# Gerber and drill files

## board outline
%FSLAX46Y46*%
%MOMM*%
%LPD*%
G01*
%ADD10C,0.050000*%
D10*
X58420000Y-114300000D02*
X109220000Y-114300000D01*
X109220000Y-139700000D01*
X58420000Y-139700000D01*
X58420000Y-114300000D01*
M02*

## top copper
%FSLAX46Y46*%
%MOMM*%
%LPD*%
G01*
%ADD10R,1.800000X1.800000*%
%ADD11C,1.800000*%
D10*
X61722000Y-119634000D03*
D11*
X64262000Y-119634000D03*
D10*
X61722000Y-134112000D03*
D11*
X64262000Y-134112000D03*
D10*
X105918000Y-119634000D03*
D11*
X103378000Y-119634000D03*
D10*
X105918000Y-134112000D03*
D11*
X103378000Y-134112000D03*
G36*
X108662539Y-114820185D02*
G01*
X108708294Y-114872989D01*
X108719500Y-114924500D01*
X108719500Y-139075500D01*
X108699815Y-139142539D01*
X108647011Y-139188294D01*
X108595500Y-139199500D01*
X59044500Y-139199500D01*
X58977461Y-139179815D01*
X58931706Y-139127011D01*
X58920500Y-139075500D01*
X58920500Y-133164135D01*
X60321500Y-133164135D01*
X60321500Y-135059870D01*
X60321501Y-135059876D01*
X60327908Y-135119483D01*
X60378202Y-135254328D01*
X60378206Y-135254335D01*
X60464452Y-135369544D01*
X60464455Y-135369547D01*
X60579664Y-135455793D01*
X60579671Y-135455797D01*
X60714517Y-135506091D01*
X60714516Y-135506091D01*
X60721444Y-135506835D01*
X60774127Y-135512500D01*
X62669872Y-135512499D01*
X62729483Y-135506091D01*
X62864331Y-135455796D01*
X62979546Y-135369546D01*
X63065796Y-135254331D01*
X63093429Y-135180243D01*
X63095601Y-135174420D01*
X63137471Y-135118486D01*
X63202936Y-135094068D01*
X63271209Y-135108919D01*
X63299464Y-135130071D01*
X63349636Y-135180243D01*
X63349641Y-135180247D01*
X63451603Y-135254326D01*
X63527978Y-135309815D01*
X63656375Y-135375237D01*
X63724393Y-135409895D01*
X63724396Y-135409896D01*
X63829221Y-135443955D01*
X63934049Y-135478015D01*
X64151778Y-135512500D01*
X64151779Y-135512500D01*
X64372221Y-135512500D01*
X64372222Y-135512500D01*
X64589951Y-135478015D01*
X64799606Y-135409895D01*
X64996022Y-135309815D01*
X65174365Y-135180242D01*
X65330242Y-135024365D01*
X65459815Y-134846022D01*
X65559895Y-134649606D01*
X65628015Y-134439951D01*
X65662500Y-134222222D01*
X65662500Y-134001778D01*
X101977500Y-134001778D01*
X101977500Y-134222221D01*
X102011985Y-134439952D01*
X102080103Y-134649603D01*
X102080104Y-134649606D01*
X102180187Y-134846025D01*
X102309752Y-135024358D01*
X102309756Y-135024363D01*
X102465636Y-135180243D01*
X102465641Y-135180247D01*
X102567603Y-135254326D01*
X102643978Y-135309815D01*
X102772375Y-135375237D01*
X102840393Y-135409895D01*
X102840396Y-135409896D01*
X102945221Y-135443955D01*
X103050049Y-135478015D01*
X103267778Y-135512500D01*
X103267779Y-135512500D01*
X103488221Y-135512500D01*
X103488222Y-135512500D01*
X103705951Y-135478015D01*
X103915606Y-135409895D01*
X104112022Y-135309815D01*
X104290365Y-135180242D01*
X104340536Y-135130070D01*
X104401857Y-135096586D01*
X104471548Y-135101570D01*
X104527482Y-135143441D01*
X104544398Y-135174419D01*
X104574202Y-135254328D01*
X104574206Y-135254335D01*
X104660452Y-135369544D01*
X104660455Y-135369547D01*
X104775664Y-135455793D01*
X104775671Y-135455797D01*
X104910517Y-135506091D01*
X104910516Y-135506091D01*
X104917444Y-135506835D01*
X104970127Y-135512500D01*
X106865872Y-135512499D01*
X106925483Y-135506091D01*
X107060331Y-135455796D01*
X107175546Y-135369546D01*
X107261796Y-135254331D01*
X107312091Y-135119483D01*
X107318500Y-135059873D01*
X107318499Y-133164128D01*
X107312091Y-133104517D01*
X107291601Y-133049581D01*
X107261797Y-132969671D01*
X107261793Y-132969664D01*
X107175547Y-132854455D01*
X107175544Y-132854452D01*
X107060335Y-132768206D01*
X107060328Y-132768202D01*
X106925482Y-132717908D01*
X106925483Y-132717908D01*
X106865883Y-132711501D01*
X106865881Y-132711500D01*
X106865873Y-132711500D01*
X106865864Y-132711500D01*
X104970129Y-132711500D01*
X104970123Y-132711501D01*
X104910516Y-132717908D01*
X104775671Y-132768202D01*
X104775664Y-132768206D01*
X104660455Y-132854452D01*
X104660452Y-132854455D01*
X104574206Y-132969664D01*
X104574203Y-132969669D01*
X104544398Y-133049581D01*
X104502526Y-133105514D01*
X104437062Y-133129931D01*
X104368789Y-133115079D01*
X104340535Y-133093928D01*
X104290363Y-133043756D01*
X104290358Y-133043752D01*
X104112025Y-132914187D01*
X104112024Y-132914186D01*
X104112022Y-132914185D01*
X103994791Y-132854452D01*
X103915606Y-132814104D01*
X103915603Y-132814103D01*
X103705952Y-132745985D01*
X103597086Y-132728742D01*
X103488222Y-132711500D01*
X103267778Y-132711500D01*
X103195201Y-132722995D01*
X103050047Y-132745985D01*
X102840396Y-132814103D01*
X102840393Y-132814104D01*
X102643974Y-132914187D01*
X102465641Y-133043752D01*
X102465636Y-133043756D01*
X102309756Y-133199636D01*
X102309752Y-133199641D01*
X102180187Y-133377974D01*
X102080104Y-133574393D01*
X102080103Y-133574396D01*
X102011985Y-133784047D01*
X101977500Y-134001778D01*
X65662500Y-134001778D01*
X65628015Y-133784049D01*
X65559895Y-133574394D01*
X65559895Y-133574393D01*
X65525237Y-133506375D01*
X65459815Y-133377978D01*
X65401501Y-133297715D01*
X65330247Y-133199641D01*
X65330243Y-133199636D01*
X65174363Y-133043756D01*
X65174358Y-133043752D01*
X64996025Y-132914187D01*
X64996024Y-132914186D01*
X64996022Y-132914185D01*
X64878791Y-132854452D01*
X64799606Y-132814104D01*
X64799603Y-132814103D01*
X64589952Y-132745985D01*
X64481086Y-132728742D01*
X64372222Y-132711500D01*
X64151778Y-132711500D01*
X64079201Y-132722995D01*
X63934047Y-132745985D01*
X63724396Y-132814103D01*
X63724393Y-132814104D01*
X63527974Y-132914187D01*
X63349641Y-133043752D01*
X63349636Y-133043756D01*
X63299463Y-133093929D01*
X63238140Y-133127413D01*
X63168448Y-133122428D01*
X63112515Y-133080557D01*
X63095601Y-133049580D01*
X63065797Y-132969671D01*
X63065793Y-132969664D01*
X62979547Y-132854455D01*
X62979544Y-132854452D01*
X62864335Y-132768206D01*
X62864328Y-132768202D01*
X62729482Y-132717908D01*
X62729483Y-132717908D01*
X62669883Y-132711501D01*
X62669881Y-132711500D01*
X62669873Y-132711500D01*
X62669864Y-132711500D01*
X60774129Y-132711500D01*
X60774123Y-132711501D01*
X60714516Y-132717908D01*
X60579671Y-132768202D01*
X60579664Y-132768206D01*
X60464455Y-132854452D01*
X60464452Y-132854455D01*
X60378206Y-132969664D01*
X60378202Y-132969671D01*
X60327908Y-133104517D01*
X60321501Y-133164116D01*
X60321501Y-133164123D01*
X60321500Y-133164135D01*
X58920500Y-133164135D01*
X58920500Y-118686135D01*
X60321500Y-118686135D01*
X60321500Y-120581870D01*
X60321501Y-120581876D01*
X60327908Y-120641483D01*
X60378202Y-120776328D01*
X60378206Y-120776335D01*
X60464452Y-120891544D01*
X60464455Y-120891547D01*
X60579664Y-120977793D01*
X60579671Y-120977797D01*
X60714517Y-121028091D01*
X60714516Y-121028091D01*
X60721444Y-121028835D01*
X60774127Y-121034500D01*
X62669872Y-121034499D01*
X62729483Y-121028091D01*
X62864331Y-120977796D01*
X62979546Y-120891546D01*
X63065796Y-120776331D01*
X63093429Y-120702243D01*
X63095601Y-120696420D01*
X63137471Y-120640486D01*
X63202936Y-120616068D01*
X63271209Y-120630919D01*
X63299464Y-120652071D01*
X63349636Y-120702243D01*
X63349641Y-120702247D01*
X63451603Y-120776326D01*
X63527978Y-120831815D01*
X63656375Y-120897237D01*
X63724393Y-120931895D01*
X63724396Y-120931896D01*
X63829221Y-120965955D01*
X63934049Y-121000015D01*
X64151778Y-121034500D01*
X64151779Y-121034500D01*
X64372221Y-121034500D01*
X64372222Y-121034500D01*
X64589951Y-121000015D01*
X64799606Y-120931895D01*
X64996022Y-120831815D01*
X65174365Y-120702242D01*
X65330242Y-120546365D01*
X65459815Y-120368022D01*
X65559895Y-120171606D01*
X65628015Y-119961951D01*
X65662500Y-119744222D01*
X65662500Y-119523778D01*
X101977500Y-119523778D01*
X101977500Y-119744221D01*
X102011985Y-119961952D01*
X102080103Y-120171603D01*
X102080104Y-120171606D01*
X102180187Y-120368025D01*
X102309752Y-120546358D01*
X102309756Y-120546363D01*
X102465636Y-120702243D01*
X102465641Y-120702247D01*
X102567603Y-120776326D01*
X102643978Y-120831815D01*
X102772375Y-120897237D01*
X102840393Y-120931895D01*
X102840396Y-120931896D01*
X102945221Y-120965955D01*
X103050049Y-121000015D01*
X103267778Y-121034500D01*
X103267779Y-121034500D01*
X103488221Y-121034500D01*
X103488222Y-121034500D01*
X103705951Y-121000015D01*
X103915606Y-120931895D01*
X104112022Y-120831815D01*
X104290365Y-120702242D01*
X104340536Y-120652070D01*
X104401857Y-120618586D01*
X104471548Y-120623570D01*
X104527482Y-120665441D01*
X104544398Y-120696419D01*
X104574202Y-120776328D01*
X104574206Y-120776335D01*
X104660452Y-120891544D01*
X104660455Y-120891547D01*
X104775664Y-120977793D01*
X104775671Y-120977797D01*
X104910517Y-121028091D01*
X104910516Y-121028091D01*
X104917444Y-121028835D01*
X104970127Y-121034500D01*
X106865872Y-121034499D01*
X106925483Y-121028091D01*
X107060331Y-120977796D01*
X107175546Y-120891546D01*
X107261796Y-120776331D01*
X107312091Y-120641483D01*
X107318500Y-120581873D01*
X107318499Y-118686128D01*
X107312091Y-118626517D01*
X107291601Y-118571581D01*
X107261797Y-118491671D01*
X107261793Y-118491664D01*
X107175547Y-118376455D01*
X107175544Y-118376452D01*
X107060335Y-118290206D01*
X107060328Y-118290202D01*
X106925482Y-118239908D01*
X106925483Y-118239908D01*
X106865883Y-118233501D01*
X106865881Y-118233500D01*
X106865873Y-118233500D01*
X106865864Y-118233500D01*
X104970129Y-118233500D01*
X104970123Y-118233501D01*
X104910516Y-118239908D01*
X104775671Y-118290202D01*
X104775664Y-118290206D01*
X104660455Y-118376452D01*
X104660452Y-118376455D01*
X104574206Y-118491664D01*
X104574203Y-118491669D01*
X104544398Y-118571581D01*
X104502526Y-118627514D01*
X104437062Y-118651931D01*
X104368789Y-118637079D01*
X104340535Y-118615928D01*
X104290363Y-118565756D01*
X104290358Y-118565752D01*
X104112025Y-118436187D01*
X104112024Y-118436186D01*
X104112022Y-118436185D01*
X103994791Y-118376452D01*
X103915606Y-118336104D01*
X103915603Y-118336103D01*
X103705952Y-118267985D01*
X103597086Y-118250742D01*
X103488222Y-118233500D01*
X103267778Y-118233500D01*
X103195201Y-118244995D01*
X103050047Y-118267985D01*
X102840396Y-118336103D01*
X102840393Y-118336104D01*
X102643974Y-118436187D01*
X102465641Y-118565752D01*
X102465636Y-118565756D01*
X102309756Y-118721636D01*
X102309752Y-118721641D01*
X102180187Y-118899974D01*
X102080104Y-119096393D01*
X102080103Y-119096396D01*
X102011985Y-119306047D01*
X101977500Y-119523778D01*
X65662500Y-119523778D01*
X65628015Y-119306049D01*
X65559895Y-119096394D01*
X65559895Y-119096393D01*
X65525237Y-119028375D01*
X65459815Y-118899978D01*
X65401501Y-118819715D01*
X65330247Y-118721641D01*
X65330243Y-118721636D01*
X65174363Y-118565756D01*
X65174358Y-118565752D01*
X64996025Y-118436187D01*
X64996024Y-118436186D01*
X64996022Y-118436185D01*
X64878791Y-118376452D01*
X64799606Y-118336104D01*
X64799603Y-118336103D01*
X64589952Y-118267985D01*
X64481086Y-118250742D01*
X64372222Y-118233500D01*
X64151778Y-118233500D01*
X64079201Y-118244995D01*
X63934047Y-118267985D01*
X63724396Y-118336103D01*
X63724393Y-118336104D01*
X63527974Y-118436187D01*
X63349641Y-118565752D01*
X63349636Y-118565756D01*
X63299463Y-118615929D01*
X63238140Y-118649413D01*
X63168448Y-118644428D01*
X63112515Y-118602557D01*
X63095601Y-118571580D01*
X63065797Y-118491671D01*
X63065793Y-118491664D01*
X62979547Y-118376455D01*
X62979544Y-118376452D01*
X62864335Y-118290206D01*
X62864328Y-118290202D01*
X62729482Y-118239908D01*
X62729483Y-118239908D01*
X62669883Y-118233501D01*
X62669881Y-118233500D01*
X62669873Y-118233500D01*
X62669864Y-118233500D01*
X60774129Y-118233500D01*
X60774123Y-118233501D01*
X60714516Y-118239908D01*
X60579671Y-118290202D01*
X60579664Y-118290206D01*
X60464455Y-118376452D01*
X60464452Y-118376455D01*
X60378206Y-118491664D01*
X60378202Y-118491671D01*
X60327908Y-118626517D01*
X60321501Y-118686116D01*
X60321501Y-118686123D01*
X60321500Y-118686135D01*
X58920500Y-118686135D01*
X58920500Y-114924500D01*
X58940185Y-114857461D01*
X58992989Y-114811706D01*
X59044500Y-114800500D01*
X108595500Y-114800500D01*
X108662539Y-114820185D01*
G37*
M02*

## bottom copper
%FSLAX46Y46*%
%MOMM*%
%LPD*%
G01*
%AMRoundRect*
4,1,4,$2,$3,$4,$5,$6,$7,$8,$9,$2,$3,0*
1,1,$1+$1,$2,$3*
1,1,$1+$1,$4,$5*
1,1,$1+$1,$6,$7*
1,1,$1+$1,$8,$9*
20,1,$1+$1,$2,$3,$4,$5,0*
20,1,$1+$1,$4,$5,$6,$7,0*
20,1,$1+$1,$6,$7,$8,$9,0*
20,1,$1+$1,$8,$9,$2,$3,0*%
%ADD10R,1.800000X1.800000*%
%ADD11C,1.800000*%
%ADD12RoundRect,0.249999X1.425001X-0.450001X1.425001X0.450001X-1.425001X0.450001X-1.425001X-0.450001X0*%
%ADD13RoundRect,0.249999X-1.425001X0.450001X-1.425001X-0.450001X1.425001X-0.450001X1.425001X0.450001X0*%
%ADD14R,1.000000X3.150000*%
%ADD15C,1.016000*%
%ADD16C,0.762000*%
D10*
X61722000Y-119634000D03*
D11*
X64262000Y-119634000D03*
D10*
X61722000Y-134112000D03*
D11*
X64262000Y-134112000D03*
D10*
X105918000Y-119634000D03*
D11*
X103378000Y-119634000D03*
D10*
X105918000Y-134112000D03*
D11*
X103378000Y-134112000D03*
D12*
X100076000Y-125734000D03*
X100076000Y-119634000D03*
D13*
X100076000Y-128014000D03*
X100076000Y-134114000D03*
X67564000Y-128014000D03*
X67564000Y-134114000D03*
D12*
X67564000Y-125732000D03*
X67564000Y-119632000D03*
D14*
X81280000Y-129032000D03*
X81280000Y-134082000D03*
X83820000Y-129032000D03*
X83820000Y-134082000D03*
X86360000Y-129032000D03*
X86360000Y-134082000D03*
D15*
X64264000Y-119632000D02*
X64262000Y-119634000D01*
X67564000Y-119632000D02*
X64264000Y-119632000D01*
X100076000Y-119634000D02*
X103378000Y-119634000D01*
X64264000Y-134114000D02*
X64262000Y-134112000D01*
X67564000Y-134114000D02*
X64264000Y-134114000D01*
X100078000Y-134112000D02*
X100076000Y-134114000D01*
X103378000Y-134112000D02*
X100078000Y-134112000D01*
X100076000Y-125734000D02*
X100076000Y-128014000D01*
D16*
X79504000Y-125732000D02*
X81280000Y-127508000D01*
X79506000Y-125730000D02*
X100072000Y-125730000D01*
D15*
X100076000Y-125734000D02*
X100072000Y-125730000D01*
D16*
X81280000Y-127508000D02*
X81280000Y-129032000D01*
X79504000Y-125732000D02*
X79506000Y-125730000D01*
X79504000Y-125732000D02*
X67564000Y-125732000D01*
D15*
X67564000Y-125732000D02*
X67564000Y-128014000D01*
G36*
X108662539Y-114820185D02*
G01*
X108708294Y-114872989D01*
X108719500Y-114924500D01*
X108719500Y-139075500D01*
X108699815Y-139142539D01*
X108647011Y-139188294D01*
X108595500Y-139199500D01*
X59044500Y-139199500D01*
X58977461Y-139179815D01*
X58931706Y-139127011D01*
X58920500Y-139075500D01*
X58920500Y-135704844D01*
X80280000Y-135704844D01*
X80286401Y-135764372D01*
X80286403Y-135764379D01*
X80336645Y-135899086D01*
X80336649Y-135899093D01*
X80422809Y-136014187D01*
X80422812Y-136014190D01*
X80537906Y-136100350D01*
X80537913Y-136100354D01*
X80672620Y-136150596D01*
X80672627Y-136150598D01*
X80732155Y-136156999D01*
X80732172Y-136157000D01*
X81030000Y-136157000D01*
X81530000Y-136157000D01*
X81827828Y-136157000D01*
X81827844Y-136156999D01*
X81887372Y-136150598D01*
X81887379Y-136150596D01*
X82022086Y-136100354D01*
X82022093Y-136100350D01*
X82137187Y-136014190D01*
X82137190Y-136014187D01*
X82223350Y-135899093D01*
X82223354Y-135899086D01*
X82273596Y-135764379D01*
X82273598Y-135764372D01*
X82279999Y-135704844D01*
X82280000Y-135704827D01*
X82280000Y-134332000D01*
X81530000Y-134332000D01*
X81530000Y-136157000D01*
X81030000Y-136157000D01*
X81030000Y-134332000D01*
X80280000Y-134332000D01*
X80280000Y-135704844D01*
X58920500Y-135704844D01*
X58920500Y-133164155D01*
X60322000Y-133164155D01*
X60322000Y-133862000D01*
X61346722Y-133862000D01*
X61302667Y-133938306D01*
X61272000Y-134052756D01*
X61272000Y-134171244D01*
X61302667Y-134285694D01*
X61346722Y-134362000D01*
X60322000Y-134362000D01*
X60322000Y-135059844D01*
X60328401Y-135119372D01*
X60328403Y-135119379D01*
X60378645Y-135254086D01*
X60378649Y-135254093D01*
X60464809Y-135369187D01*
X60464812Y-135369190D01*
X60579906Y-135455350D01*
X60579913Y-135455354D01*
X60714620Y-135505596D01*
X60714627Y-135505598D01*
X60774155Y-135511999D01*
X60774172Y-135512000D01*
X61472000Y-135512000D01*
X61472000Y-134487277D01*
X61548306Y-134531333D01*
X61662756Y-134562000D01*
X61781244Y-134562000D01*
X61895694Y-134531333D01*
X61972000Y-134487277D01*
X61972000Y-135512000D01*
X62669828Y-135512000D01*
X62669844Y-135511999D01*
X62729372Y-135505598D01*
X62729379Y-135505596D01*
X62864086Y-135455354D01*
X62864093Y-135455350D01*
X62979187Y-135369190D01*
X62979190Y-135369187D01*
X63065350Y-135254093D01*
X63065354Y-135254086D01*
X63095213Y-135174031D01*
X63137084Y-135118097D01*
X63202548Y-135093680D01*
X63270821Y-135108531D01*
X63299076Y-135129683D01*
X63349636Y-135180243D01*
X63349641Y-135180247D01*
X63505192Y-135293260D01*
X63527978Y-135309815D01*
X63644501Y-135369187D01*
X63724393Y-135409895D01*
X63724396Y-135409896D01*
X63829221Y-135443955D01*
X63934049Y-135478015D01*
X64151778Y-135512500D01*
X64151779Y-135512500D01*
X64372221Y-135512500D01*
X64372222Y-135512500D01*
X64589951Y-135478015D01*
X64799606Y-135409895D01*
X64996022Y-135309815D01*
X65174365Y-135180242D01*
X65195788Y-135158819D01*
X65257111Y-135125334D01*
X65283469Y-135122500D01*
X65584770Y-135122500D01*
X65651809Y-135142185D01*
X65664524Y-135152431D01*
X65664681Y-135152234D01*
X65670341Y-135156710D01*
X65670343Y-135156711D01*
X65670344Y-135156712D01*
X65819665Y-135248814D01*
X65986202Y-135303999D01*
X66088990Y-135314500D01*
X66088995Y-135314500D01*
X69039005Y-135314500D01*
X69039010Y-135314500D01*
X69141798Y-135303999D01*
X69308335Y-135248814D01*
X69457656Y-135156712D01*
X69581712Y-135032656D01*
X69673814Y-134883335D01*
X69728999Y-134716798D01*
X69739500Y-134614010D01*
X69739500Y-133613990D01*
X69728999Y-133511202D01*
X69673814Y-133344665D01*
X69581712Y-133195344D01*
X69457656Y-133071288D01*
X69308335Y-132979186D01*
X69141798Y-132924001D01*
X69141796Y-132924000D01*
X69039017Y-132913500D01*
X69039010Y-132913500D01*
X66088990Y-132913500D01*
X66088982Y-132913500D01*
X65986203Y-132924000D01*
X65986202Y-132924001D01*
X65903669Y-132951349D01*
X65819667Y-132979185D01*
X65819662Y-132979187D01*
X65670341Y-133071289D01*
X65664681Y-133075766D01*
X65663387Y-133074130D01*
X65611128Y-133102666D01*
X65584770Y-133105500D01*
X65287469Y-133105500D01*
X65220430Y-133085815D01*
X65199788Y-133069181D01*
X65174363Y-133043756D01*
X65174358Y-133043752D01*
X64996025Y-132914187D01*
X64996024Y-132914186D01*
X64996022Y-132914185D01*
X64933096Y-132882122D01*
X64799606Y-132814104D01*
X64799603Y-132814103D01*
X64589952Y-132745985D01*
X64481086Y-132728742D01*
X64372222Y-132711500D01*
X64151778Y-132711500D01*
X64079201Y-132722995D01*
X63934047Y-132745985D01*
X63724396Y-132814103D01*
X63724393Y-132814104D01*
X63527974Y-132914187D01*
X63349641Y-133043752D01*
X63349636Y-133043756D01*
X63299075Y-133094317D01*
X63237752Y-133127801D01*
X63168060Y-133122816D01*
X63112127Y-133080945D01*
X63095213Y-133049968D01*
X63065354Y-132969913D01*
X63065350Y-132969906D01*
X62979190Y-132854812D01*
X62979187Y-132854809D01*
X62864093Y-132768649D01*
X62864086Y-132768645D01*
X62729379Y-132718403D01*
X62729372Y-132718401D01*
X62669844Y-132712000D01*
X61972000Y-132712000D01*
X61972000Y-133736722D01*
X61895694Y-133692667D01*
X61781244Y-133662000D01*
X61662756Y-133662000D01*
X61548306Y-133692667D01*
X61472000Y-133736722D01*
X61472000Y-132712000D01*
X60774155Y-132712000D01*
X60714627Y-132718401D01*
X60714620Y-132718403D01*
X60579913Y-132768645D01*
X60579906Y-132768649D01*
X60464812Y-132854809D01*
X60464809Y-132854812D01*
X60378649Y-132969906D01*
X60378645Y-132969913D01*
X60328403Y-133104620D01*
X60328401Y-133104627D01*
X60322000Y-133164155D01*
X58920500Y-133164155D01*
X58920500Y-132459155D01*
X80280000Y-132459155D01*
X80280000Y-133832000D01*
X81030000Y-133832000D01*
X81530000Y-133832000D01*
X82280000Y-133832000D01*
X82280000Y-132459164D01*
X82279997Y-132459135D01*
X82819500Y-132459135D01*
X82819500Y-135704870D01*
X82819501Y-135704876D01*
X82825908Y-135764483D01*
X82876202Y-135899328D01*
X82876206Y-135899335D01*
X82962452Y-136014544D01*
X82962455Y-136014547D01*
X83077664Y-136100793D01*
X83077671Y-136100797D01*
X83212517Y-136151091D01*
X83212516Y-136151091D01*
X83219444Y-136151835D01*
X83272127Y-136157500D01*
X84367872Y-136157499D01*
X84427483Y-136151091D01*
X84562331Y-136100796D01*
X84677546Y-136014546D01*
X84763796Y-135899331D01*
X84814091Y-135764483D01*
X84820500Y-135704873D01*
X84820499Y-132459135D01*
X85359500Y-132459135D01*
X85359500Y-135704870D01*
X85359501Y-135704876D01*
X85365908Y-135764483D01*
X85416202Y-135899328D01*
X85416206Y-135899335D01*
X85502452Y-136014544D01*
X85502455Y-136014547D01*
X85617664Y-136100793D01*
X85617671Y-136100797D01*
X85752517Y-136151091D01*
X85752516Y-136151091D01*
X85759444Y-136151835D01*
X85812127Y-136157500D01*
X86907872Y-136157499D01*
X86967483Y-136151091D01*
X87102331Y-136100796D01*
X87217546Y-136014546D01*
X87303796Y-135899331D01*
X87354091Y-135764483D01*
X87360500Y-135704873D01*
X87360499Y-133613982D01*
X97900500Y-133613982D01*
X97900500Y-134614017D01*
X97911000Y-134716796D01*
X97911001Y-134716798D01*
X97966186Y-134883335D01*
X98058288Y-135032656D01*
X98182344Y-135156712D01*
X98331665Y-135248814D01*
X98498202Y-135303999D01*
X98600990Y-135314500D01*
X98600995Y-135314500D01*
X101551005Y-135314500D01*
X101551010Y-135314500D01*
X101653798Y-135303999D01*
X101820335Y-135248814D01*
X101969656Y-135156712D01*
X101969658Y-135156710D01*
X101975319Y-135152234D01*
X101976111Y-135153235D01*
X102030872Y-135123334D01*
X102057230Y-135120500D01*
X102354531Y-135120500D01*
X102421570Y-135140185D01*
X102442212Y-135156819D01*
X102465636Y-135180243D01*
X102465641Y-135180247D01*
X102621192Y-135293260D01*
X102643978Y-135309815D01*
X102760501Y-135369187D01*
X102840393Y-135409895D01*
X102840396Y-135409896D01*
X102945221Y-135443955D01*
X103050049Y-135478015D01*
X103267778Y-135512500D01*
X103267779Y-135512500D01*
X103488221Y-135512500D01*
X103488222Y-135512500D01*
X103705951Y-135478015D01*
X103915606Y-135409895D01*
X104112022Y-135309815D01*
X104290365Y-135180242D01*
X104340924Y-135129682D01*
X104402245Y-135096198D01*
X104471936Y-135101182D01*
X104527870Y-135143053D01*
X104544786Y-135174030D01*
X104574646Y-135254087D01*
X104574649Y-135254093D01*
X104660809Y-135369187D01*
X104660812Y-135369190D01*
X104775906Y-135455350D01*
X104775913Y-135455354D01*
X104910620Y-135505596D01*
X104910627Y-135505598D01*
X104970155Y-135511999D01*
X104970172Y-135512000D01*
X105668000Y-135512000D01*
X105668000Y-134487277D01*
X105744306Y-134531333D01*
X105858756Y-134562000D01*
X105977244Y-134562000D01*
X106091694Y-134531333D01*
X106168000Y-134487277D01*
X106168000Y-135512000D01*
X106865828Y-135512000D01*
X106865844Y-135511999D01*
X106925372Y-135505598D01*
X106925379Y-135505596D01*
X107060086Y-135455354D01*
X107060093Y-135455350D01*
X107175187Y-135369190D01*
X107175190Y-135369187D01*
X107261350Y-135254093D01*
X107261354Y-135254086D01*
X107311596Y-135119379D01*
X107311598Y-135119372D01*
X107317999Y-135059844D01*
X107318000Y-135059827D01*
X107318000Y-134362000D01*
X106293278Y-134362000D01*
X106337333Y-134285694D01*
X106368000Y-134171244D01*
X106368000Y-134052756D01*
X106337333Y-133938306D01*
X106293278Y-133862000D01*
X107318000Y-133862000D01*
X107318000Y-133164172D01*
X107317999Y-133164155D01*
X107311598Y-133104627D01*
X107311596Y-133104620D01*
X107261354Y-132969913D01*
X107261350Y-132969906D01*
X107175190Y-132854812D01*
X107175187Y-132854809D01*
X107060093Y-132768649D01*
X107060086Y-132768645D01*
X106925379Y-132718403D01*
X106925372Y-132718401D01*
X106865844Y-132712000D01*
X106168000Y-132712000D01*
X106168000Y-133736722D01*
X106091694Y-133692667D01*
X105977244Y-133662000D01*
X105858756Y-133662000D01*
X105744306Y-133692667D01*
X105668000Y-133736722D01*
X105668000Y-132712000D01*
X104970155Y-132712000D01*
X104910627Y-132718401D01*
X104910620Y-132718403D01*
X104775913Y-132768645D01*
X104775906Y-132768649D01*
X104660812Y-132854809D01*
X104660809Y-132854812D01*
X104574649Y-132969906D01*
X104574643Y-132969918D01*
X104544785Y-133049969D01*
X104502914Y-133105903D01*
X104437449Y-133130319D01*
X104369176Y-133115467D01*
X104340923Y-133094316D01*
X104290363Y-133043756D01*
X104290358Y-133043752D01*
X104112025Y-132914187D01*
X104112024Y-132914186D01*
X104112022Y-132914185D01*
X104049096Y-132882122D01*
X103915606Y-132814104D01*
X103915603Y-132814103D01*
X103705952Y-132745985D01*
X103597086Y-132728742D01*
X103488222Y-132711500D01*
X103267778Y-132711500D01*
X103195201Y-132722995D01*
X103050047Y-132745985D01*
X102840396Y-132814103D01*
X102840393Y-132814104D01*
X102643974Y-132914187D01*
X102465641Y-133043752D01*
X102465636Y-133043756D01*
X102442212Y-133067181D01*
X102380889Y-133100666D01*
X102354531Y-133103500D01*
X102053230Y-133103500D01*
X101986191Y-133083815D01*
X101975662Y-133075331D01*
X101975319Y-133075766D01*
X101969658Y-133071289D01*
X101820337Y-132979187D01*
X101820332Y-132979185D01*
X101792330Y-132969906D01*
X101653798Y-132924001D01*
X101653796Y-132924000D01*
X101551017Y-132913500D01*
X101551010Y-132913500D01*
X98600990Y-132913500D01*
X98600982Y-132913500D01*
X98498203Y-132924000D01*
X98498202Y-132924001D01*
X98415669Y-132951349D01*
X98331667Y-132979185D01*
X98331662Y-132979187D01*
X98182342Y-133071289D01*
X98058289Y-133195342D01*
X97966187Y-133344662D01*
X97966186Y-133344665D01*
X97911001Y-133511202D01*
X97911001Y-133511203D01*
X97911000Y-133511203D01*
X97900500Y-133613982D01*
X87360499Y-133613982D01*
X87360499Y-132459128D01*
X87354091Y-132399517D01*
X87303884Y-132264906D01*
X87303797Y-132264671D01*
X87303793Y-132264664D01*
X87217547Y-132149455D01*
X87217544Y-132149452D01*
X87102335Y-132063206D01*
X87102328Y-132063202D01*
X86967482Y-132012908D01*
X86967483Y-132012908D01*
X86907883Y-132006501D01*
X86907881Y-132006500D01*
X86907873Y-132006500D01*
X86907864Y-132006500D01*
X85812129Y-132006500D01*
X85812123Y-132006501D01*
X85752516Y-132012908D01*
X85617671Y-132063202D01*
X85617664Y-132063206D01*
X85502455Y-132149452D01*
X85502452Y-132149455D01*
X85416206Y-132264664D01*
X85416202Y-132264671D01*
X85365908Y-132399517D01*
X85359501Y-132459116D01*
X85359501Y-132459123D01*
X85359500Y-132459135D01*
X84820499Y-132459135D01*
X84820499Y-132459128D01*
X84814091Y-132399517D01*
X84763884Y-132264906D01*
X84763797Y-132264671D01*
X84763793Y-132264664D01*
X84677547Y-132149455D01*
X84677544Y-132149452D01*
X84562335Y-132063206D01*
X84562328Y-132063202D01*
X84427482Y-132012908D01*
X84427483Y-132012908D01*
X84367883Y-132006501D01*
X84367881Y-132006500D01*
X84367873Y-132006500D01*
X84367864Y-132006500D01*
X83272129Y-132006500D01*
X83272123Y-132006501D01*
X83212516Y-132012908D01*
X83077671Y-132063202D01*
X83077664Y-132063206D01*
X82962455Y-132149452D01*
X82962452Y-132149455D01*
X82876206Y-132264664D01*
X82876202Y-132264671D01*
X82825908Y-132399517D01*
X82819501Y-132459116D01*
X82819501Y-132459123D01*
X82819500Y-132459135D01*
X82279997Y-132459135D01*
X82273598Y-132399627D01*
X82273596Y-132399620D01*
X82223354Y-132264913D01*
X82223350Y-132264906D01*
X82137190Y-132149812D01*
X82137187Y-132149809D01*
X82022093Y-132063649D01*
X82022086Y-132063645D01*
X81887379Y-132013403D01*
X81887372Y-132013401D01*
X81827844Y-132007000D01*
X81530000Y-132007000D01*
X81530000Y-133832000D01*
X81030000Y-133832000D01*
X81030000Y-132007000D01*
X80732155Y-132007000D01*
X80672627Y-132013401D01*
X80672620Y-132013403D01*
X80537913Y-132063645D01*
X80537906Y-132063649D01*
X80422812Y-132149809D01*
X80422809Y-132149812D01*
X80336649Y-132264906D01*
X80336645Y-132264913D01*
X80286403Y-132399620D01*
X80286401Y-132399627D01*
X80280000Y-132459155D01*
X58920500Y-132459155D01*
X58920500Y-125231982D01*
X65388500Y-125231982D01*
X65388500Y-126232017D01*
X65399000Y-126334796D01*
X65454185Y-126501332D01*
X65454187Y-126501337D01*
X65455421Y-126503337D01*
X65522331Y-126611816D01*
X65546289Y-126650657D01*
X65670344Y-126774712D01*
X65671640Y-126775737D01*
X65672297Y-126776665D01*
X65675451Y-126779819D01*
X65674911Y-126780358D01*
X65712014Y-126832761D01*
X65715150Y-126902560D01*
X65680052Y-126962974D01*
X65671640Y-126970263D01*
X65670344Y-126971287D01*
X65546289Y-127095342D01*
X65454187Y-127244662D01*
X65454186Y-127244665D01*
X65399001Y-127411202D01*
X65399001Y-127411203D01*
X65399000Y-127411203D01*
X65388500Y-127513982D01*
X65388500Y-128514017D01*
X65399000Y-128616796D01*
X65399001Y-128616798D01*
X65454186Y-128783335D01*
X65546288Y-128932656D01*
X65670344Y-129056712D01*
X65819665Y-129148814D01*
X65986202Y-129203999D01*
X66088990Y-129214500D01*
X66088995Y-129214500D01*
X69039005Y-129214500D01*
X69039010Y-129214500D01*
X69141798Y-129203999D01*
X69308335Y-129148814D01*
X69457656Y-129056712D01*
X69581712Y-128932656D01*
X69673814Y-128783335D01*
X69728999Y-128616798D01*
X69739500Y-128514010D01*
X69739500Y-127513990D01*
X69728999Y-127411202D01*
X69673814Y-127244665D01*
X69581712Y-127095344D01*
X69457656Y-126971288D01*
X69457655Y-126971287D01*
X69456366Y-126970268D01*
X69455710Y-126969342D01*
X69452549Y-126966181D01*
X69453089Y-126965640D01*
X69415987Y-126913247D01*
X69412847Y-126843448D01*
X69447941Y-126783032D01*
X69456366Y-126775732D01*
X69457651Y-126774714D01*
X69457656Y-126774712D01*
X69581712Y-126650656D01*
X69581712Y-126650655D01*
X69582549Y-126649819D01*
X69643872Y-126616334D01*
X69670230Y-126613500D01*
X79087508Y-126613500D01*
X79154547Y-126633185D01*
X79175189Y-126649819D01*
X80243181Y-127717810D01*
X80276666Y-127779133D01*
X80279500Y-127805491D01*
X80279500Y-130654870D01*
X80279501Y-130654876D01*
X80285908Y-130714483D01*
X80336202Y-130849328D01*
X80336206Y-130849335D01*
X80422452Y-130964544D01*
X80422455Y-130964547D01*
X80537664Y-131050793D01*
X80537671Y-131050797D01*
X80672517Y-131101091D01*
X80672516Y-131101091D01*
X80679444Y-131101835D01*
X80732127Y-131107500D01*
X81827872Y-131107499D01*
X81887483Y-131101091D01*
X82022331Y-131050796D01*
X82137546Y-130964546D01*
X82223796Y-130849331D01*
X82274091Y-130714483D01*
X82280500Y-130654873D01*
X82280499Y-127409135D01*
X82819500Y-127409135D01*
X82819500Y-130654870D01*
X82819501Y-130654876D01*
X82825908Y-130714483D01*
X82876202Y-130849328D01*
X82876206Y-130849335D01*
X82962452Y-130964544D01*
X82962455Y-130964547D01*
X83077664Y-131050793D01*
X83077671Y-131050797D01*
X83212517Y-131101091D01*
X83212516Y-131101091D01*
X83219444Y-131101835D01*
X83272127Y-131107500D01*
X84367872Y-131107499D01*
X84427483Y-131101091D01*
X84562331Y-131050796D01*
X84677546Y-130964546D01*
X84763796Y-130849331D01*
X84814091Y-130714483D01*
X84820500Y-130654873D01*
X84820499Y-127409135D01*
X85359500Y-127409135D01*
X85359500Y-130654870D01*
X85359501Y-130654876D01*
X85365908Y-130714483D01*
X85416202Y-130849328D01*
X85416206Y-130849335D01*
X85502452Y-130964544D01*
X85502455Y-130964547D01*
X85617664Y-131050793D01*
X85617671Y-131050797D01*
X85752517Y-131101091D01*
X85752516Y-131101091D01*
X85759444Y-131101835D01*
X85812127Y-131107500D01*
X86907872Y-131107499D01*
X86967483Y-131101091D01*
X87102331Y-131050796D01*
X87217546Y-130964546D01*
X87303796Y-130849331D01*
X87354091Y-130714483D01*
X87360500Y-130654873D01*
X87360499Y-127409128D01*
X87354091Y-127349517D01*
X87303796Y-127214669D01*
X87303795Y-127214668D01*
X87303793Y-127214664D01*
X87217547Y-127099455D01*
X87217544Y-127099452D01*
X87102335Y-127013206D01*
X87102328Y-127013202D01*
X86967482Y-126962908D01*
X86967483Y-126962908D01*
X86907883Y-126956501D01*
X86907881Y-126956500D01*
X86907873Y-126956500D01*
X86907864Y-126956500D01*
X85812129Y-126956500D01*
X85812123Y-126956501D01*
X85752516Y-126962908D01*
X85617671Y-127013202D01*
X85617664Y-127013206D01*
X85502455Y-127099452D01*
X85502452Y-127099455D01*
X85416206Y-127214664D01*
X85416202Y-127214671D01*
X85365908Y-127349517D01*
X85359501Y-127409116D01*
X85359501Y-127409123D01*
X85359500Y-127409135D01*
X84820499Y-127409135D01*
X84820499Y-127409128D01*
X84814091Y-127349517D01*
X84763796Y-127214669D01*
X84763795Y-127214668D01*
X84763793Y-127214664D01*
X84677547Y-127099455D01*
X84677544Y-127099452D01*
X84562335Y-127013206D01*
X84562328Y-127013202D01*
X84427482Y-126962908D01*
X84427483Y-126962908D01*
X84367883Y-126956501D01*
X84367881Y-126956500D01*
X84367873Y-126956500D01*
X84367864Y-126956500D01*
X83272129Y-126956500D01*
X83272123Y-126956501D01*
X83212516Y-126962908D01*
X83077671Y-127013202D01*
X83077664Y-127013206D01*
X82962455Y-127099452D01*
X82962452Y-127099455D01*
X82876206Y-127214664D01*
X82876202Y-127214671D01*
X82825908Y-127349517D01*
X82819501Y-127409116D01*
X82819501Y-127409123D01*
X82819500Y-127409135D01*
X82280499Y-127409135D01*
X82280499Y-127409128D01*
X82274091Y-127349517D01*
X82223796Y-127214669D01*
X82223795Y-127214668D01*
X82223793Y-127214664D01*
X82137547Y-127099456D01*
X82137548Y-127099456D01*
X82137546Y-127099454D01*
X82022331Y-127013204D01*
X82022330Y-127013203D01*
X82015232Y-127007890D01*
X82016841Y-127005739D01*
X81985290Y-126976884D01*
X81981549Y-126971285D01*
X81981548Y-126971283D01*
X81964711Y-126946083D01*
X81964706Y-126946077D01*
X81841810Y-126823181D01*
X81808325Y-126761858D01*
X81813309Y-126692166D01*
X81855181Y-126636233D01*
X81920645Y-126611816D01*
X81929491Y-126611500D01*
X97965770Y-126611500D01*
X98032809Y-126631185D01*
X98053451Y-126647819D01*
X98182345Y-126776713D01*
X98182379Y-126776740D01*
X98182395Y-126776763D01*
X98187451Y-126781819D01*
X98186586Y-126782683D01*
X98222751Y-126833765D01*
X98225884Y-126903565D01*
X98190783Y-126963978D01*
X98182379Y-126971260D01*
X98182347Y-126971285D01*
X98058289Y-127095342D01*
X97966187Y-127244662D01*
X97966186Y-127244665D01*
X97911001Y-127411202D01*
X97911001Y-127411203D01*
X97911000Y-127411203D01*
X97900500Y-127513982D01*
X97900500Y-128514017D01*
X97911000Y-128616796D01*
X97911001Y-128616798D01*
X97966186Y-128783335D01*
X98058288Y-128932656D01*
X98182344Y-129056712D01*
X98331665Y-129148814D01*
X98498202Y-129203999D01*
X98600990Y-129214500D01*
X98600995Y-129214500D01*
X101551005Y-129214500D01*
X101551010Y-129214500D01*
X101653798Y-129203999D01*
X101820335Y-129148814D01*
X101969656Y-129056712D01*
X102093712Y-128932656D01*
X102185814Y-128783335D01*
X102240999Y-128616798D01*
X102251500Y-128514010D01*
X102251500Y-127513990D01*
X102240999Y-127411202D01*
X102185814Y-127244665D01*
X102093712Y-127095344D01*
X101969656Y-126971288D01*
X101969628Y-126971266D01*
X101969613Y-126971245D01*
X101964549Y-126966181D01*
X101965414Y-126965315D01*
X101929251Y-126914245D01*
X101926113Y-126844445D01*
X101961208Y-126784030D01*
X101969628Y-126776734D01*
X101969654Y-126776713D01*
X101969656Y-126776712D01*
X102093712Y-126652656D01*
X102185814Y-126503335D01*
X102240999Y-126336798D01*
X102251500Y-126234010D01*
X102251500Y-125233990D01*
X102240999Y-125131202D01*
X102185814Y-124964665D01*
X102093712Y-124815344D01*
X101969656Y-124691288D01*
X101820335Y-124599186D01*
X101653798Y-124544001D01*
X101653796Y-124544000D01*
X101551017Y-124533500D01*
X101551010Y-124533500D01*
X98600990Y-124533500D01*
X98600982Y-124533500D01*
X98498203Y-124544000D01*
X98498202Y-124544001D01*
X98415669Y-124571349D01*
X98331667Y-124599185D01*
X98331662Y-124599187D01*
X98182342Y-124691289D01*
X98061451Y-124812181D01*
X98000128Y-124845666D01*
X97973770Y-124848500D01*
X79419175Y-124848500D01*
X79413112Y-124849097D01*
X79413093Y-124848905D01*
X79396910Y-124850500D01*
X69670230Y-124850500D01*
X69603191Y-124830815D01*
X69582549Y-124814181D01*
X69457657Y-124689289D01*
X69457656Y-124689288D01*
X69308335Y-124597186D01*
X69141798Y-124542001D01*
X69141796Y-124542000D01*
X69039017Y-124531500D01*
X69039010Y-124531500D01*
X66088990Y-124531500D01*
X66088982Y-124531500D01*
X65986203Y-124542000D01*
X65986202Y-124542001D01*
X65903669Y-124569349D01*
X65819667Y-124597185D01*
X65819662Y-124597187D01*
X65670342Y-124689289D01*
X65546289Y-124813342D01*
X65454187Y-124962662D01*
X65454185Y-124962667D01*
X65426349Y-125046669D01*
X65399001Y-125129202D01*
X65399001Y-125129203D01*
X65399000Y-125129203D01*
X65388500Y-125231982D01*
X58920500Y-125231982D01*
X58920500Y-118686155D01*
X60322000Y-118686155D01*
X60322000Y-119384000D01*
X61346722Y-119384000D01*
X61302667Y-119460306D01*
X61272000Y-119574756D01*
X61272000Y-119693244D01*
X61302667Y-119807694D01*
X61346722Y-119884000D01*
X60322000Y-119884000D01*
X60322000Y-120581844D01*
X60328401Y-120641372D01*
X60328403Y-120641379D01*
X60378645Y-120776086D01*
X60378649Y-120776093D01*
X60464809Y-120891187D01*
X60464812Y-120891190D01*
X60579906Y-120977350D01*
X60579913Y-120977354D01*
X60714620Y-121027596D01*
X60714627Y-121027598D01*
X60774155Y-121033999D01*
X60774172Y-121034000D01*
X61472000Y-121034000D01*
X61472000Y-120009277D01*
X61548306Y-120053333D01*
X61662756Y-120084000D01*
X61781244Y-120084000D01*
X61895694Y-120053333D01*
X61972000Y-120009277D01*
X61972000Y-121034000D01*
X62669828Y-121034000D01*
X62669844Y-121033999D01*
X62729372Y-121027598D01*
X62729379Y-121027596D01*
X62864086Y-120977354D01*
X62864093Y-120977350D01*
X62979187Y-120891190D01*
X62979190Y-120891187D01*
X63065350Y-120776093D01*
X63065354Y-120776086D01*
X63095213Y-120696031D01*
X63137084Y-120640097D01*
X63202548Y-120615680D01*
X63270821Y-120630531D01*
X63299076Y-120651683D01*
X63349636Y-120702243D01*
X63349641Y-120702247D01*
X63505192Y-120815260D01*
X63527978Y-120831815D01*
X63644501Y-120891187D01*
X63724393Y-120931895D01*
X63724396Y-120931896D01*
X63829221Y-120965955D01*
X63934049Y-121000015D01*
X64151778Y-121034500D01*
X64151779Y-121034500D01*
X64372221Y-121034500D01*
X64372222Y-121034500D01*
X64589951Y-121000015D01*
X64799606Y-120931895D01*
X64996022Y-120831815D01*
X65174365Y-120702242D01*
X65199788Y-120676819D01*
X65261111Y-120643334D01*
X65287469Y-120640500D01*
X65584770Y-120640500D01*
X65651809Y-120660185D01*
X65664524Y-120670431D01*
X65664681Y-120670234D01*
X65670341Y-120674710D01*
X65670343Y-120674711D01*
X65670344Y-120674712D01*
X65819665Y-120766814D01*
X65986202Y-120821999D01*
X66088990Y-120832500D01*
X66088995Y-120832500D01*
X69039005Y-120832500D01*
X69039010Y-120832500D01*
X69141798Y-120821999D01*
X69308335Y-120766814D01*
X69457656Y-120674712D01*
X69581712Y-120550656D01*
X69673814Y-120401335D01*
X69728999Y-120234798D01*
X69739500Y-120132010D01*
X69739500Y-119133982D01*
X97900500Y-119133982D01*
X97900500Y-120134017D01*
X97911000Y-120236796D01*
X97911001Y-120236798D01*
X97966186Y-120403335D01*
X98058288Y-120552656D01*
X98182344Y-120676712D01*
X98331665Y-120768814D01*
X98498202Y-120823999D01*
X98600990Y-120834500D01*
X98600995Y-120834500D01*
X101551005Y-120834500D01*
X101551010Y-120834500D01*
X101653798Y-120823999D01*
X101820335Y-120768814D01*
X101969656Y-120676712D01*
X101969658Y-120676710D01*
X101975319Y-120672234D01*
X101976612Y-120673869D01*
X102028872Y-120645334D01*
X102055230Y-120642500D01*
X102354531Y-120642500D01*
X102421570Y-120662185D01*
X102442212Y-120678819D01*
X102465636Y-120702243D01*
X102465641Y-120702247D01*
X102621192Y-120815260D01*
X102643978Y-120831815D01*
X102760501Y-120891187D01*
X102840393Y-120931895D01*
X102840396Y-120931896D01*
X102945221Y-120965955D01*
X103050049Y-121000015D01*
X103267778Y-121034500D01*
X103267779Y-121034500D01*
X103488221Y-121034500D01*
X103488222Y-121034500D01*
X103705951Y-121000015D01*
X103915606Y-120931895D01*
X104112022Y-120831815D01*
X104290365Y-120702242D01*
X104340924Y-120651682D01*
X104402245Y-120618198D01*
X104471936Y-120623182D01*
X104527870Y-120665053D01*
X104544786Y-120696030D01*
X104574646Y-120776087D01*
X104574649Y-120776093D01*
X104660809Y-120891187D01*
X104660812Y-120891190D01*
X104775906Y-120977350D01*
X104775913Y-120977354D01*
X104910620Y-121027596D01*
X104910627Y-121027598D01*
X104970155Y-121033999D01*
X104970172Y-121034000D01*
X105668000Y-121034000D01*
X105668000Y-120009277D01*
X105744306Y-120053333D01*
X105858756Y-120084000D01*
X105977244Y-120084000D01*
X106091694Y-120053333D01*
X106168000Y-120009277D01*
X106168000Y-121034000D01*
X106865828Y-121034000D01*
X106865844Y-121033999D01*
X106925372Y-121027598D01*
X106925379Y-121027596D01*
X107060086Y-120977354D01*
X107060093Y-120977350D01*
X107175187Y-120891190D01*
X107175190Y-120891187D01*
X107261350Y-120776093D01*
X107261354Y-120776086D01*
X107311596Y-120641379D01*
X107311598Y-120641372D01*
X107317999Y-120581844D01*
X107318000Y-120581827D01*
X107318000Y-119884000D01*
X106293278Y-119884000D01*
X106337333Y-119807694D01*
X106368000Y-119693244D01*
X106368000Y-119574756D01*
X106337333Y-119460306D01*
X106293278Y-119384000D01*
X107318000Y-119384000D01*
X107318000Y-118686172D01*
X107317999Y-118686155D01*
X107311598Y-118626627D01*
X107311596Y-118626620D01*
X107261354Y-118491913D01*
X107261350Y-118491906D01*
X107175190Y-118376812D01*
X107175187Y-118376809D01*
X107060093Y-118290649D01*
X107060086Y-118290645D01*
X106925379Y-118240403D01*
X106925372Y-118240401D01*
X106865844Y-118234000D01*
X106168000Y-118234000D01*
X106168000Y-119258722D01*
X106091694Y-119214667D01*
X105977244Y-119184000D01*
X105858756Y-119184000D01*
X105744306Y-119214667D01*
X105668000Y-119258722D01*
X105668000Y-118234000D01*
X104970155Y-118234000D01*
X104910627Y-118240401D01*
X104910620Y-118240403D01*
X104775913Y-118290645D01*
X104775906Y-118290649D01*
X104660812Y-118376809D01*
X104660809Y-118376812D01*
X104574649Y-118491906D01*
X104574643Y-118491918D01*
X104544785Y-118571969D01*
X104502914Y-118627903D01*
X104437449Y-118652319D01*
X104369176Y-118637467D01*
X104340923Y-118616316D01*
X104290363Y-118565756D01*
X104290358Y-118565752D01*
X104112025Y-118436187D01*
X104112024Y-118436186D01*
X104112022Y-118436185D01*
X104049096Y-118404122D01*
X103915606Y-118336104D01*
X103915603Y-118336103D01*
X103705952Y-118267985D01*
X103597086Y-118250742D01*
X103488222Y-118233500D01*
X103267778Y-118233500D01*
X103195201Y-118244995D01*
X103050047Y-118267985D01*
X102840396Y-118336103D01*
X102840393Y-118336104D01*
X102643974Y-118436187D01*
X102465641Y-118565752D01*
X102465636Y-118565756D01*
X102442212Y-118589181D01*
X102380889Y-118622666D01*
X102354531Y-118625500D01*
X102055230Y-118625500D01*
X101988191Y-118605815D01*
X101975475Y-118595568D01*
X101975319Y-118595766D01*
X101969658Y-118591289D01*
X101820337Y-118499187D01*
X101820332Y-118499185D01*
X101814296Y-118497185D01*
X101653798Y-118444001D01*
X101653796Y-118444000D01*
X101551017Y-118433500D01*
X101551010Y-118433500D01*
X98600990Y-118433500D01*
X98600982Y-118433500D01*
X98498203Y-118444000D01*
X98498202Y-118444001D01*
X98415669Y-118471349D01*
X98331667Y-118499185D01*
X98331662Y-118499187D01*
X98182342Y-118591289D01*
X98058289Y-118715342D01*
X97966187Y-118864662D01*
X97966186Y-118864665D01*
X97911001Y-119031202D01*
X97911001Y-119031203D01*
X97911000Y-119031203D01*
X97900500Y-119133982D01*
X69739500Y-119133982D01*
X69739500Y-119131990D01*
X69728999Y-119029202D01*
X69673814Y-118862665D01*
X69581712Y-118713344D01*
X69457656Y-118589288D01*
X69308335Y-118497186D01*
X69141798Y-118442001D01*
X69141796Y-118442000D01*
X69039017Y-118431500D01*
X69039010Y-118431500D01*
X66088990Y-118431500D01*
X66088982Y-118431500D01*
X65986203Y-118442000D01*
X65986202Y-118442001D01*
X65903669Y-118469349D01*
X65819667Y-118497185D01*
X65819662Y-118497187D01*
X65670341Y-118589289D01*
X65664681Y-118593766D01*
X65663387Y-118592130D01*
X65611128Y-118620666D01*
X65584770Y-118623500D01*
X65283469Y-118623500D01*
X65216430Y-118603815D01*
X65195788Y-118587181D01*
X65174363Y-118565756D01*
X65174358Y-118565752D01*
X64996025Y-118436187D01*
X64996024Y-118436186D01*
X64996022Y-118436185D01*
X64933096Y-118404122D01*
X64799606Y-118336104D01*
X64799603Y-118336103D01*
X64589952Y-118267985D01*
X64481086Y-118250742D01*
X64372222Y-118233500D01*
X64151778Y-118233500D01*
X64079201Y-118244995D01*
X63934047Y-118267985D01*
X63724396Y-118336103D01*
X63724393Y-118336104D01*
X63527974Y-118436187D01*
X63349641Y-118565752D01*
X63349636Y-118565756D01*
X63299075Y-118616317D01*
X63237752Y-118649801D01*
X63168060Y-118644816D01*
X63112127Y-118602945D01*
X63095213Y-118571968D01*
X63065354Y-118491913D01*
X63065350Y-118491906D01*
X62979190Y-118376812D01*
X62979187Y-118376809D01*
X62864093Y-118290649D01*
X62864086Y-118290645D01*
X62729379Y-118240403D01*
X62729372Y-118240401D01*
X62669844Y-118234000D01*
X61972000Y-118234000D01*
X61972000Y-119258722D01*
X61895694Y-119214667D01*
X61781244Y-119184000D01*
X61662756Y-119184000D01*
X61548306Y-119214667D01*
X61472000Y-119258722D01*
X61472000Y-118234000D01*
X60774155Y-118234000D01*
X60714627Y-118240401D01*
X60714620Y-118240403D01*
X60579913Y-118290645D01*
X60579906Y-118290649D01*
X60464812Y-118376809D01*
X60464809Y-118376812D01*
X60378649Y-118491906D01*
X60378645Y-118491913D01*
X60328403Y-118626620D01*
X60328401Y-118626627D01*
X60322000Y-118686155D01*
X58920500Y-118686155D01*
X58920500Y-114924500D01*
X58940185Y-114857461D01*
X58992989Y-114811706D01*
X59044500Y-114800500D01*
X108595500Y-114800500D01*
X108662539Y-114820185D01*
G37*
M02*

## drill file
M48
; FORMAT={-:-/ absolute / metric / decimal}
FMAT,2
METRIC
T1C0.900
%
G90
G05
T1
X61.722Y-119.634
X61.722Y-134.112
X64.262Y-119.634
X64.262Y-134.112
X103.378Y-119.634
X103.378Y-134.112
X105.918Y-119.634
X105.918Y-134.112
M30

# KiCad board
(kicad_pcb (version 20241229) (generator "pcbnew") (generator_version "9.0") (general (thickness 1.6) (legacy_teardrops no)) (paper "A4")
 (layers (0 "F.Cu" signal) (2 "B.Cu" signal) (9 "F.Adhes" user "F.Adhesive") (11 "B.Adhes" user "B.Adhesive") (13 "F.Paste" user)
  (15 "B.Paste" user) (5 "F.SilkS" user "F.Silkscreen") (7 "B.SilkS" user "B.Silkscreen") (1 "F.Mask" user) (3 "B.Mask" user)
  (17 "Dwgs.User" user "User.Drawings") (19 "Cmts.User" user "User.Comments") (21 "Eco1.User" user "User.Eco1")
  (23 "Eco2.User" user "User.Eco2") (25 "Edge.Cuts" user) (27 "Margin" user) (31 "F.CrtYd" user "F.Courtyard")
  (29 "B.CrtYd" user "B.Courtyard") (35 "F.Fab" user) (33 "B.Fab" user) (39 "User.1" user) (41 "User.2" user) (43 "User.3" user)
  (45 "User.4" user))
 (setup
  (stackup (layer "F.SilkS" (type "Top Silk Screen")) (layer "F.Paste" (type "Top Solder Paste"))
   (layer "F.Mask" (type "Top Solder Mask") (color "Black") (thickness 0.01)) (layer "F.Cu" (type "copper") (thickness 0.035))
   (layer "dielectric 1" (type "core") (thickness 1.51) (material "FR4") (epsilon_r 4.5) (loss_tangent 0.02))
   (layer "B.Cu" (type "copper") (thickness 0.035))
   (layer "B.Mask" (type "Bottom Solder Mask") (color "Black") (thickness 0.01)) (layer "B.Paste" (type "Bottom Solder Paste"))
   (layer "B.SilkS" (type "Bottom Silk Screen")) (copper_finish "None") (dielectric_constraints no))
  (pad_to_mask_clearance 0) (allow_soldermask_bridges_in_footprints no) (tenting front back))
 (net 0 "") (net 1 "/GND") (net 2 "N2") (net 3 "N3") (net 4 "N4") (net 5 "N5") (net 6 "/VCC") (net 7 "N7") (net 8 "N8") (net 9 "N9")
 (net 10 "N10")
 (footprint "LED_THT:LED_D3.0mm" (layer "F.Cu") (at 61.722 119.634)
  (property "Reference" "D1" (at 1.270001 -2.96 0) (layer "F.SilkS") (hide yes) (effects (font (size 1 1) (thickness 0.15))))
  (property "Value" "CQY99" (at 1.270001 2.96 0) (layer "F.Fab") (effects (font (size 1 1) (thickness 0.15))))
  (pad "1" thru_hole rect (at 0 0) (size 1.8 1.8) (drill 0.9) (layers "*.Cu" "*.Mask") (remove_unused_layers no) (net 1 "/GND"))
  (pad "2" thru_hole circle (at 2.54 0) (size 1.8 1.8) (drill 0.9) (layers "*.Cu" "*.Mask") (remove_unused_layers no) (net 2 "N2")))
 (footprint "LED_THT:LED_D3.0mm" (layer "F.Cu") (at 61.722 134.112)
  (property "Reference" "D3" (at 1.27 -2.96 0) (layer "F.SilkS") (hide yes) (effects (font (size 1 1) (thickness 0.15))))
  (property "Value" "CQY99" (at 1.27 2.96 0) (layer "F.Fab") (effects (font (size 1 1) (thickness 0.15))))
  (pad "1" thru_hole rect (at 0 0) (size 1.8 1.8) (drill 0.9) (layers "*.Cu" "*.Mask") (remove_unused_layers no) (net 1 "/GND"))
  (pad "2" thru_hole circle (at 2.54 0) (size 1.8 1.8) (drill 0.9) (layers "*.Cu" "*.Mask") (remove_unused_layers no) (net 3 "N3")))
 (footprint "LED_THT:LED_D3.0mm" (layer "F.Cu") (at 105.918 119.634 180)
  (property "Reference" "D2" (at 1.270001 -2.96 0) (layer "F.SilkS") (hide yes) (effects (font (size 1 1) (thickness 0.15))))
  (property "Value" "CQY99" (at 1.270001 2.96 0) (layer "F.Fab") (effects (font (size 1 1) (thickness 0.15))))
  (pad "1" thru_hole rect (at 0 0 180) (size 1.8 1.8) (drill 0.9) (layers "*.Cu" "*.Mask") (remove_unused_layers no) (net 1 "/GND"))
  (pad "2" thru_hole circle (at 2.54 0 180) (size 1.8 1.8) (drill 0.9) (layers "*.Cu" "*.Mask") (remove_unused_layers no) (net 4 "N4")))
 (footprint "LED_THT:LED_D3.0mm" (layer "F.Cu") (at 105.918 134.112 180)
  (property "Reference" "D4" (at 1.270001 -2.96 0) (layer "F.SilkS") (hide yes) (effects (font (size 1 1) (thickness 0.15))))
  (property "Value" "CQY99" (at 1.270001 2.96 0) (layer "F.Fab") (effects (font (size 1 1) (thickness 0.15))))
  (pad "1" thru_hole rect (at 0 0 180) (size 1.8 1.8) (drill 0.9) (layers "*.Cu" "*.Mask") (remove_unused_layers no) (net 1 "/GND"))
  (pad "2" thru_hole circle (at 2.54 0 180) (size 1.8 1.8) (drill 0.9) (layers "*.Cu" "*.Mask") (remove_unused_layers no) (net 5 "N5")))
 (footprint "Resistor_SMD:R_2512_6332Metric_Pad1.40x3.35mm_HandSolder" (layer "B.Cu") (at 100.076 122.684 90)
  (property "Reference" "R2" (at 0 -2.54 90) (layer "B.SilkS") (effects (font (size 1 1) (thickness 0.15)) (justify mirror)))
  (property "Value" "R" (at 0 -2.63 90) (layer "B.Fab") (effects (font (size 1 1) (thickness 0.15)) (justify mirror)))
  (pad "1" smd roundrect (at -3.05 0 90) (size 1.4 3.35) (layers "B.Cu" "B.Mask" "B.Paste") (roundrect_rratio 0.178571) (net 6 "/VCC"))
  (pad "2" smd roundrect (at 3.05 0 90) (size 1.4 3.35) (layers "B.Cu" "B.Mask" "B.Paste") (roundrect_rratio 0.178571) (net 4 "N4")))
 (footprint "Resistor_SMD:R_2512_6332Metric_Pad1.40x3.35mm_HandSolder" (layer "B.Cu") (at 100.076 131.064 -90)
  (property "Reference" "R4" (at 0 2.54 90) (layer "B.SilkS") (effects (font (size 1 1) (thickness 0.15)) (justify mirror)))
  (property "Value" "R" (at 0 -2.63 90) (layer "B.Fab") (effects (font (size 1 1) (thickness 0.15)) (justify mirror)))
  (pad "1" smd roundrect (at -3.05 0 270) (size 1.4 3.35) (layers "B.Cu" "B.Mask" "B.Paste") (roundrect_rratio 0.178571) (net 6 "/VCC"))
  (pad "2" smd roundrect (at 3.05 0 270) (size 1.4 3.35) (layers "B.Cu" "B.Mask" "B.Paste") (roundrect_rratio 0.178571) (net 5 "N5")))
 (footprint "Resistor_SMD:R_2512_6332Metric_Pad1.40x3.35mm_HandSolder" (layer "B.Cu") (at 67.564 131.064 -90)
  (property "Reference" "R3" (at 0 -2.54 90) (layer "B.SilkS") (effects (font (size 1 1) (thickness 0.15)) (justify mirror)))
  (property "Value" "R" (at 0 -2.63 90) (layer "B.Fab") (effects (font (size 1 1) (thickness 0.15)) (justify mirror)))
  (pad "1" smd roundrect (at -3.05 0 270) (size 1.4 3.35) (layers "B.Cu" "B.Mask" "B.Paste") (roundrect_rratio 0.178571) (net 6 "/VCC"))
  (pad "2" smd roundrect (at 3.05 0 270) (size 1.4 3.35) (layers "B.Cu" "B.Mask" "B.Paste") (roundrect_rratio 0.178571) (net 3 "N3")))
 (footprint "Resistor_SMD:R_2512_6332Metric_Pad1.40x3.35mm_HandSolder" (layer "B.Cu") (at 67.564 122.682 90)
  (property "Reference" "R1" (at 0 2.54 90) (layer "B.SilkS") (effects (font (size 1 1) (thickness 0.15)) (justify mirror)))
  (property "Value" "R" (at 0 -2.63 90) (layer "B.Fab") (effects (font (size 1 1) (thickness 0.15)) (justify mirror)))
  (pad "1" smd roundrect (at -3.05 0 90) (size 1.4 3.35) (layers "B.Cu" "B.Mask" "B.Paste") (roundrect_rratio 0.178571) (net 6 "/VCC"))
  (pad "2" smd roundrect (at 3.05 0 90) (size 1.4 3.35) (layers "B.Cu" "B.Mask" "B.Paste") (roundrect_rratio 0.178571) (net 2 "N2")))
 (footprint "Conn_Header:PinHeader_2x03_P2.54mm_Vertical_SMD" (layer "B.Cu") (at 83.82 131.557 -90)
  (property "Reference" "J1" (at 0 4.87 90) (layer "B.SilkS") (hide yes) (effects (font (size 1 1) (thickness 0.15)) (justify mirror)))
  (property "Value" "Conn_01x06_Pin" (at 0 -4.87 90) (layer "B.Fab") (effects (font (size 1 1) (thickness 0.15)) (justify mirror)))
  (pad "1" smd rect (at -2.525 2.54 270) (size 3.15 1) (layers "B.Cu" "B.Mask" "B.Paste") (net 6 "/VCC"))
  (pad "2" smd rect (at 2.525 2.54 270) (size 3.15 1) (layers "B.Cu" "B.Mask" "B.Paste") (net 1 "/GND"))
  (pad "3" smd rect (at -2.525 0 270) (size 3.15 1) (layers "B.Cu" "B.Mask" "B.Paste") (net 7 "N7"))
  (pad "4" smd rect (at 2.525 0 270) (size 3.15 1) (layers "B.Cu" "B.Mask" "B.Paste") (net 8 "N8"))
  (pad "5" smd rect (at -2.525 -2.54 270) (size 3.15 1) (layers "B.Cu" "B.Mask" "B.Paste") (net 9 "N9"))
  (pad "6" smd rect (at 2.525 -2.54 270) (size 3.15 1) (layers "B.Cu" "B.Mask" "B.Paste") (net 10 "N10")))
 (gr_rect (start 58.42 114.3) (end 109.22 139.7) (stroke (width 0.05) (type default)) (fill no) (layer "Edge.Cuts"))
 (segment (start 64.264 119.632) (end 64.262 119.634) (width 1.016) (layer "B.Cu") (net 2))
 (segment (start 67.564 119.632) (end 64.264 119.632) (width 1.016) (layer "B.Cu") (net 2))
 (segment (start 100.076 119.634) (end 103.378 119.634) (width 1.016) (layer "B.Cu") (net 4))
 (segment (start 64.264 134.114) (end 64.262 134.112) (width 1.016) (layer "B.Cu") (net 3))
 (segment (start 67.564 134.114) (end 64.264 134.114) (width 1.016) (layer "B.Cu") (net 3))
 (segment (start 100.078 134.112) (end 100.076 134.114) (width 1.016) (layer "B.Cu") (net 5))
 (segment (start 103.378 134.112) (end 100.078 134.112) (width 1.016) (layer "B.Cu") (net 5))
 (segment (start 100.076 125.734) (end 100.076 128.014) (width 1.016) (layer "B.Cu") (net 6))
 (segment (start 79.504 125.732) (end 81.28 127.508) (width 0.762) (layer "B.Cu") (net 6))
 (segment (start 79.506 125.73) (end 100.072 125.73) (width 0.762) (layer "B.Cu") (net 6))
 (segment (start 100.076 125.734) (end 100.072 125.73) (width 1.016) (layer "B.Cu") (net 6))
 (segment (start 81.28 127.508) (end 81.28 129.032) (width 0.762) (layer "B.Cu") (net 6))
 (segment (start 79.504 125.732) (end 79.506 125.73) (width 0.762) (layer "B.Cu") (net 6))
 (segment (start 79.504 125.732) (end 67.564 125.732) (width 0.762) (layer "B.Cu") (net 6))
 (segment (start 67.564 125.732) (end 67.564 128.014) (width 1.016) (layer "B.Cu") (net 6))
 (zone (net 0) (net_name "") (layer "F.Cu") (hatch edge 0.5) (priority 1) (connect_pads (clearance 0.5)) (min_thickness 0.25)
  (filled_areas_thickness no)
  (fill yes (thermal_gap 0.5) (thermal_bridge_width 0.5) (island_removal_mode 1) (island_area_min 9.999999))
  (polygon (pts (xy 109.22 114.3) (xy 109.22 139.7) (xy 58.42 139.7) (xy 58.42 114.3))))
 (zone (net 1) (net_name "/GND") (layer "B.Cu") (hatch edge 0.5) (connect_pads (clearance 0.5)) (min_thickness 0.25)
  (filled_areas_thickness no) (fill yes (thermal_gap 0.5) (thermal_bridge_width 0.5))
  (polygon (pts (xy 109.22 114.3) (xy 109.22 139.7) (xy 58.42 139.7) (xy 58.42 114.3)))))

